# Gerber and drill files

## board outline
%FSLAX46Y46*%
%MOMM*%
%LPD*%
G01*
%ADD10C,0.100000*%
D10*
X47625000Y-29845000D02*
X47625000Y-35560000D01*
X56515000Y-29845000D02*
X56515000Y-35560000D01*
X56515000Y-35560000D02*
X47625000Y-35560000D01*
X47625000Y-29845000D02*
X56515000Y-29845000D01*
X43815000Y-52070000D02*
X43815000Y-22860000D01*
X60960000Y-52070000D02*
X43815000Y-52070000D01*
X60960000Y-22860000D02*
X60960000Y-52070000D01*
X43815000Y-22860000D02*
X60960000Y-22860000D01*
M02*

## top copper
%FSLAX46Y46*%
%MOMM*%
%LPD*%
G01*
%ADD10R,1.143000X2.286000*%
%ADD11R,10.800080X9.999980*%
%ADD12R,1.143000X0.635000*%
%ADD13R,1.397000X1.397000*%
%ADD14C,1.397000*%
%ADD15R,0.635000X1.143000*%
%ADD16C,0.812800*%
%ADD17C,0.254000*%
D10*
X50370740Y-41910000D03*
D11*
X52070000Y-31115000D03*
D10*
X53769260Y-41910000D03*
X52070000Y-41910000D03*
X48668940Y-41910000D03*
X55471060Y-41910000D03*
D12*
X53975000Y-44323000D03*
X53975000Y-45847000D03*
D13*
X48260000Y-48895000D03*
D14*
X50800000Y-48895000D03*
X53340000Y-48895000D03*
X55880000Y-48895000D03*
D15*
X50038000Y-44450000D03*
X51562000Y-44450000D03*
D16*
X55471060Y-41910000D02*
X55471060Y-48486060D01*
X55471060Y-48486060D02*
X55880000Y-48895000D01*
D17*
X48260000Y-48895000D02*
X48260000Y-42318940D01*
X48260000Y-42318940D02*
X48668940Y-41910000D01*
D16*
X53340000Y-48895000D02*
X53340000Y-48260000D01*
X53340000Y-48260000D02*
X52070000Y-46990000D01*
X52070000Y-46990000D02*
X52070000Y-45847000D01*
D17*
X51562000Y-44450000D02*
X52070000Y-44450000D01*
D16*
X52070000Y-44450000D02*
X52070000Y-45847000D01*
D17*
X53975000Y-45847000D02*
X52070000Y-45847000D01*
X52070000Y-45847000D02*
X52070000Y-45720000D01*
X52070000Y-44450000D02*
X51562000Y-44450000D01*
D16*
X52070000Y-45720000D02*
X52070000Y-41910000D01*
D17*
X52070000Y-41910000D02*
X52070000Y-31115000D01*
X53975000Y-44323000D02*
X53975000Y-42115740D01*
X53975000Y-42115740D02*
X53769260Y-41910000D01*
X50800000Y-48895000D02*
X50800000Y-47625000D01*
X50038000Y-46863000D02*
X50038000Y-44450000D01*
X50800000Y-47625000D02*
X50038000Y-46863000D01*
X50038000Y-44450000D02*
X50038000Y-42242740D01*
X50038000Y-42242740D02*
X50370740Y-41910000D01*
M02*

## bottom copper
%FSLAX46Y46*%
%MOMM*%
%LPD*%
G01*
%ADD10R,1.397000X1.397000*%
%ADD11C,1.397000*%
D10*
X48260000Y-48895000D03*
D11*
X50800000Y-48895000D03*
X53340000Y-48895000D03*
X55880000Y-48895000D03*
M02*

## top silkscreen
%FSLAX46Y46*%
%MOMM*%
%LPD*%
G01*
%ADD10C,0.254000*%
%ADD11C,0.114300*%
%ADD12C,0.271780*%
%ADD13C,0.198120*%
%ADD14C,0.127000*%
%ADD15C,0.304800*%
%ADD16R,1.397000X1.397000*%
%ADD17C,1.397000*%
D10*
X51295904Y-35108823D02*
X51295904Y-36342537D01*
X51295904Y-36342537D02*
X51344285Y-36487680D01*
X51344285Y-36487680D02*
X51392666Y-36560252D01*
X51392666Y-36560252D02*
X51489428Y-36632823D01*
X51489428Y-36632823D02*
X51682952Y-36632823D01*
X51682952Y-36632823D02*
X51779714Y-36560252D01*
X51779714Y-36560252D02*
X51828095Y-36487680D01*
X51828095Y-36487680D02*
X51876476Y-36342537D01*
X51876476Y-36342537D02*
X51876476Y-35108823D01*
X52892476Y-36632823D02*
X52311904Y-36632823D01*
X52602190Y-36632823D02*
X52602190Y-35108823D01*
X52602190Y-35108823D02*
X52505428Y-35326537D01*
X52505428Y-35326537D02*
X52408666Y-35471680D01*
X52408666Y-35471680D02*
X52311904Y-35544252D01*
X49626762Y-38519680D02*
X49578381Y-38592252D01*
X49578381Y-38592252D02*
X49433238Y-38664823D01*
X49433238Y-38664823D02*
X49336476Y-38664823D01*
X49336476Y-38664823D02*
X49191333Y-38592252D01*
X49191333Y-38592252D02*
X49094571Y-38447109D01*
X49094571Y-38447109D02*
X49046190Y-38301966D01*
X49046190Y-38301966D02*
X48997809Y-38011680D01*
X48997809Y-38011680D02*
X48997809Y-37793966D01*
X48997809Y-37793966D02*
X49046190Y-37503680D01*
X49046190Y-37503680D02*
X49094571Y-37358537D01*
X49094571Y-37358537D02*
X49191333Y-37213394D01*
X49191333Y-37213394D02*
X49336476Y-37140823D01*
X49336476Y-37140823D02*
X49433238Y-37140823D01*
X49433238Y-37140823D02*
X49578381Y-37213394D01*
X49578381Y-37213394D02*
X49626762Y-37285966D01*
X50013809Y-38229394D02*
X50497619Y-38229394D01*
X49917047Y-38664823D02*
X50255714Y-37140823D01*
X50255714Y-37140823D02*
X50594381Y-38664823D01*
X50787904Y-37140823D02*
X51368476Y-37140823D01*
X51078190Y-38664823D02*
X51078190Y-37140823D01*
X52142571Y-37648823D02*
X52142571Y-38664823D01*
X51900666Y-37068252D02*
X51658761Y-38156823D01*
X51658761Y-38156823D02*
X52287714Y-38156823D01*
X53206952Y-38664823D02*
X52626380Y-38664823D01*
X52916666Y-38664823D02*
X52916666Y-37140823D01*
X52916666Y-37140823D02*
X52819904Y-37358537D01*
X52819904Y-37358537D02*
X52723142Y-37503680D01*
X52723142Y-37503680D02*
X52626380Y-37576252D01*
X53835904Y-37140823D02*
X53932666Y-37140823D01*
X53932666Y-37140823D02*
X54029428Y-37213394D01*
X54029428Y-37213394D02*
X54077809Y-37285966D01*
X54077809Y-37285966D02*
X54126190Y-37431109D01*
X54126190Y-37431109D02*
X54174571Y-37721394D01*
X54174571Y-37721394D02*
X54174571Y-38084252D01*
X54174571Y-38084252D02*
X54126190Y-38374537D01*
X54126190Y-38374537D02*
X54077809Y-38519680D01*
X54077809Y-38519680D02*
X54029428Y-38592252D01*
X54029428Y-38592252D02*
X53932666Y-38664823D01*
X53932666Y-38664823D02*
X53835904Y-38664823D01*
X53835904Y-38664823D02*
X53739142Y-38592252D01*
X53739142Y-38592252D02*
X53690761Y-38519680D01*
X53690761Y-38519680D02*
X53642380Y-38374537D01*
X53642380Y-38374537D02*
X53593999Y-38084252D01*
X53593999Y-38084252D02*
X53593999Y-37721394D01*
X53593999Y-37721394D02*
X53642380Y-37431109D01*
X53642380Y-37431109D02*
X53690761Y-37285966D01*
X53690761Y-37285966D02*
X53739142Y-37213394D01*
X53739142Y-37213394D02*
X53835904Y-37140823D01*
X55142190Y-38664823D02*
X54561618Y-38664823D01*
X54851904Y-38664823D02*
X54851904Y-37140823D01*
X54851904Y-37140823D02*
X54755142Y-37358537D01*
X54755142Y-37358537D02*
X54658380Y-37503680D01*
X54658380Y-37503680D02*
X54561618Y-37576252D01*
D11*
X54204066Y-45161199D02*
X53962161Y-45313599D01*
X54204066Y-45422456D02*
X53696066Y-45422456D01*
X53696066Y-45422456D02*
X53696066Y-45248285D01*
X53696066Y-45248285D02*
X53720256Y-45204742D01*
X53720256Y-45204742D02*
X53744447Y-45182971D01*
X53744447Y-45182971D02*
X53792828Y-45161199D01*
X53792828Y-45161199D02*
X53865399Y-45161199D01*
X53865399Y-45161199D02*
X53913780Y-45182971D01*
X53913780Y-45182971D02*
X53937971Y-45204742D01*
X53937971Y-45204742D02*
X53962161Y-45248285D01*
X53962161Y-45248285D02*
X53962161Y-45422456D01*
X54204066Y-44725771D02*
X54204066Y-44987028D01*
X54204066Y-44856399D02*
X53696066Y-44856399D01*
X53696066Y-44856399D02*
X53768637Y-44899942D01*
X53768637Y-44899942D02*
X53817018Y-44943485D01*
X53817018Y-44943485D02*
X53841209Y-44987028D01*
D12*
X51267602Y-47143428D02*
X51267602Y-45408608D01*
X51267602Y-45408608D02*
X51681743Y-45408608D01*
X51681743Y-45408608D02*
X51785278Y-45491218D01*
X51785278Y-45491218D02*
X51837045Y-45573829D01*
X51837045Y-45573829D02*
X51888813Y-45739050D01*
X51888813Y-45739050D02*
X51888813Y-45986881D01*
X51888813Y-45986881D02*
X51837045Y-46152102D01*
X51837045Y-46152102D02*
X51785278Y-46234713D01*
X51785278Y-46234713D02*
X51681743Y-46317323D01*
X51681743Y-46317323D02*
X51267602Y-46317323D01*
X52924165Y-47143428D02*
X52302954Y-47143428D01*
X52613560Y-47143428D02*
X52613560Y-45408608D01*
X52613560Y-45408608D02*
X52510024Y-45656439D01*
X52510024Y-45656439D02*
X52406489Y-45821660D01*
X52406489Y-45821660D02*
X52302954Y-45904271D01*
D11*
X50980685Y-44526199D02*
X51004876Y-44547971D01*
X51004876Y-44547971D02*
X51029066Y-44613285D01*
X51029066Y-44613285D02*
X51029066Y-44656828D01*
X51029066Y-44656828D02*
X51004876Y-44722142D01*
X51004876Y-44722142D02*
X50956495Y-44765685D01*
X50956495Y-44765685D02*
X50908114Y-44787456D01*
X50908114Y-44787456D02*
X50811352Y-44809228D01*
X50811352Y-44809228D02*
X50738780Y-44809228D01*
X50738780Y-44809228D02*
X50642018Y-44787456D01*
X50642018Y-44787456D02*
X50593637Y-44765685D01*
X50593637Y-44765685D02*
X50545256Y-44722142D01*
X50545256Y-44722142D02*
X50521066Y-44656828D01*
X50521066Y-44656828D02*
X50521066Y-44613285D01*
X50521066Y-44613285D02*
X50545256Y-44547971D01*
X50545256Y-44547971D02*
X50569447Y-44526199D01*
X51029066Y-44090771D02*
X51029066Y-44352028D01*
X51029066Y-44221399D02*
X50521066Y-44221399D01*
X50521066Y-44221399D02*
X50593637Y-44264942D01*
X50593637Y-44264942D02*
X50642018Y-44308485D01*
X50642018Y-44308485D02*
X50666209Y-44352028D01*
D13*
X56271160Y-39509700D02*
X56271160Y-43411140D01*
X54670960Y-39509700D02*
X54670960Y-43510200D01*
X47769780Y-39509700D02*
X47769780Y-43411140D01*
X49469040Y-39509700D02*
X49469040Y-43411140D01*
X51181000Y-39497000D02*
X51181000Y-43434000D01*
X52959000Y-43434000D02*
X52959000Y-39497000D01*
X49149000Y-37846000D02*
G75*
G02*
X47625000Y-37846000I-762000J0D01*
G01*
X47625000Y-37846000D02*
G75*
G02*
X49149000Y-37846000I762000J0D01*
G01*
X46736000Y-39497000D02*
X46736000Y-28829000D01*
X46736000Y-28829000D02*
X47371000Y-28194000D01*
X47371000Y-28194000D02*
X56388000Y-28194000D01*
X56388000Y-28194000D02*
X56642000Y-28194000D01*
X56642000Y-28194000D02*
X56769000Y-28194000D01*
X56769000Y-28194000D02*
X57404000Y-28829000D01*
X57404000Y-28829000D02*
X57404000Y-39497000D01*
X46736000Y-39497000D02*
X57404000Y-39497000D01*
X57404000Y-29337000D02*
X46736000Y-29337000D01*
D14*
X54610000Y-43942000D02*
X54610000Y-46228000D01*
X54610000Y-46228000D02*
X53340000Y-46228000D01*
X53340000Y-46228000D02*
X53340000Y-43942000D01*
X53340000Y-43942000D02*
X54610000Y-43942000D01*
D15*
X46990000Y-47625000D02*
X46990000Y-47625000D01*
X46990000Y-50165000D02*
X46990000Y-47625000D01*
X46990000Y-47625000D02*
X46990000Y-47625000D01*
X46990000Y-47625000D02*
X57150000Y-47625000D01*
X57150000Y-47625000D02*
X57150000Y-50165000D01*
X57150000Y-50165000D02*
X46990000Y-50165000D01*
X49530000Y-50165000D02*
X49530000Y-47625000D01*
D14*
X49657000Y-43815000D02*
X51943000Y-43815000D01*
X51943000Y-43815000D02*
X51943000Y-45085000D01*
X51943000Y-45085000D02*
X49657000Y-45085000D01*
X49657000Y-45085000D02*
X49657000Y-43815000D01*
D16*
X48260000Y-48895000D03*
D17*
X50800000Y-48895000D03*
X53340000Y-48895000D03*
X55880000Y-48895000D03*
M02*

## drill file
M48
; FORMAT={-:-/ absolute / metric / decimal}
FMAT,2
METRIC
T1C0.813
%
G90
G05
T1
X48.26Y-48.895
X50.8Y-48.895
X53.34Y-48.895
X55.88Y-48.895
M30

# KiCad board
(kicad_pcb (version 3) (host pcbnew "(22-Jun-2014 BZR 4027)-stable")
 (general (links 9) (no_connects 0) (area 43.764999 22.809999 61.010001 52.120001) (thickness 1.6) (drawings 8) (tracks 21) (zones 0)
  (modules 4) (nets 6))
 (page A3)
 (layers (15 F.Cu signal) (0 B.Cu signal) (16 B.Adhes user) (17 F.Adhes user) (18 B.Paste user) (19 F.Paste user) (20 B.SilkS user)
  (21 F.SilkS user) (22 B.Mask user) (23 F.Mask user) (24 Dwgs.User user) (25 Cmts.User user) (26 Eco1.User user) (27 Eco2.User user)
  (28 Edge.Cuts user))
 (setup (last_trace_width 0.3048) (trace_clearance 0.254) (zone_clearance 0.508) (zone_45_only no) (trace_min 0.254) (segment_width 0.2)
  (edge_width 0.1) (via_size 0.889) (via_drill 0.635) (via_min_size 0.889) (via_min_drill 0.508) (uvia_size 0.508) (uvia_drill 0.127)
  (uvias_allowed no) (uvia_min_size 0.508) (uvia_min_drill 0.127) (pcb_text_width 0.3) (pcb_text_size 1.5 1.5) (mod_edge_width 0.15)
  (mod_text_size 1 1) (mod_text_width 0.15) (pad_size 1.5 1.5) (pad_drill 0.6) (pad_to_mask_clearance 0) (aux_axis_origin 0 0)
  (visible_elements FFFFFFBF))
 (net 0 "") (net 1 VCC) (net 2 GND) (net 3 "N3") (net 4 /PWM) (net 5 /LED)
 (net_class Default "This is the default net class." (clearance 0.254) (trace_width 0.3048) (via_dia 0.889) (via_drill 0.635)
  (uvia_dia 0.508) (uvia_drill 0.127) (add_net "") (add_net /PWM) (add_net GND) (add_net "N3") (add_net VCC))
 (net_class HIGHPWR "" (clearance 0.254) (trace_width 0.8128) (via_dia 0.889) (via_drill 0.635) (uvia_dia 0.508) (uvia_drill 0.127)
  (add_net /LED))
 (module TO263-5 (layer F.Cu) (at 52.07 41.91)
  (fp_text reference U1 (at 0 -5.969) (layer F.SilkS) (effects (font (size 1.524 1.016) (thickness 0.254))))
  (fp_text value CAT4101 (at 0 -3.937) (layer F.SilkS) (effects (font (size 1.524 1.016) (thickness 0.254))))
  (fp_line (start 4.20116 -2.4003) (end 4.20116 1.50114) (layer F.SilkS) (width 0.19812))
  (fp_line (start 2.60096 -2.4003) (end 2.60096 1.6002) (layer F.SilkS) (width 0.19812))
  (fp_line (start -4.30022 -2.4003) (end -4.30022 1.50114) (layer F.SilkS) (width 0.19812))
  (fp_line (start -2.60096 -2.4003) (end -2.60096 1.50114) (layer F.SilkS) (width 0.19812))
  (fp_line (start -0.889 -2.413) (end -0.889 1.524) (layer F.SilkS) (width 0.19812))
  (fp_line (start 0.889 1.524) (end 0.889 -2.413) (layer F.SilkS) (width 0.19812))
  (fp_circle (center -3.683 -4.064) (end -3.683 -3.302) (layer F.SilkS) (width 0.19812))
  (fp_line (start -5.334 -2.413) (end -5.334 -13.081) (layer F.SilkS) (width 0.19812))
  (fp_line (start -5.334 -13.081) (end -4.699 -13.716) (layer F.SilkS) (width 0.19812))
  (fp_line (start -4.699 -13.716) (end 4.318 -13.716) (layer F.SilkS) (width 0.19812))
  (fp_line (start 4.318 -13.716) (end 4.572 -13.716) (layer F.SilkS) (width 0.19812))
  (fp_line (start 4.572 -13.716) (end 4.699 -13.716) (layer F.SilkS) (width 0.19812))
  (fp_line (start 4.699 -13.716) (end 5.334 -13.081) (layer F.SilkS) (width 0.19812))
  (fp_line (start 5.334 -13.081) (end 5.334 -2.413) (layer F.SilkS) (width 0.19812))
  (fp_line (start -5.334 -2.413) (end 5.334 -2.413) (layer F.SilkS) (width 0.19812))
  (fp_line (start 5.334 -12.573) (end -5.334 -12.573) (layer F.SilkS) (width 0.19812))
  (pad 2 smd rect (at -1.69926 0) (size 1.143 2.286) (layers F.Cu F.Paste F.Mask) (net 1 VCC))
  (pad 3 smd rect (at 0 -10.795) (size 10.80008 9.99998) (layers F.Cu F.Paste F.Mask) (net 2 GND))
  (pad 4 smd rect (at 1.69926 0) (size 1.143 2.286) (layers F.Cu F.Paste F.Mask) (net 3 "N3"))
  (pad 3 smd rect (at 0 0) (size 1.143 2.286) (layers F.Cu F.Paste F.Mask) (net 2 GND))
  (pad 1 smd rect (at -3.40106 0) (size 1.143 2.286) (layers F.Cu F.Paste F.Mask) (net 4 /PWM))
  (pad 5 smd rect (at 3.40106 0) (size 1.143 2.286) (layers F.Cu F.Paste F.Mask) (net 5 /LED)))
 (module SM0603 (layer F.Cu) (at 53.975 45.085 270)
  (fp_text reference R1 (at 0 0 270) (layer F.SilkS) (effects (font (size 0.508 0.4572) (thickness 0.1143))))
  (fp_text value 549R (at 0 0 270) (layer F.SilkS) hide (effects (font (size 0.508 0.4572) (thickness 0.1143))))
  (fp_line (start -1.143 -0.635) (end 1.143 -0.635) (layer F.SilkS) (width 0.127))
  (fp_line (start 1.143 -0.635) (end 1.143 0.635) (layer F.SilkS) (width 0.127))
  (fp_line (start 1.143 0.635) (end -1.143 0.635) (layer F.SilkS) (width 0.127))
  (fp_line (start -1.143 0.635) (end -1.143 -0.635) (layer F.SilkS) (width 0.127))
  (pad 1 smd rect (at -0.762 0 270) (size 0.635 1.143) (layers F.Cu F.Paste F.Mask) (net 3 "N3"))
  (pad 2 smd rect (at 0.762 0 270) (size 0.635 1.143) (layers F.Cu F.Paste F.Mask) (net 2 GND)))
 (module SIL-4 (layer F.Cu) (at 52.07 48.895)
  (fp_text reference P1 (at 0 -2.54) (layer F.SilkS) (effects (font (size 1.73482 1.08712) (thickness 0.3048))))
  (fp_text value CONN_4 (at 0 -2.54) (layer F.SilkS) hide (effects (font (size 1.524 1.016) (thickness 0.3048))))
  (fp_line (start -5.08 -1.27) (end -5.08 -1.27) (layer F.SilkS) (width 0.3048))
  (fp_line (start -5.08 1.27) (end -5.08 -1.27) (layer F.SilkS) (width 0.3048))
  (fp_line (start -5.08 -1.27) (end -5.08 -1.27) (layer F.SilkS) (width 0.3048))
  (fp_line (start -5.08 -1.27) (end 5.08 -1.27) (layer F.SilkS) (width 0.3048))
  (fp_line (start 5.08 -1.27) (end 5.08 1.27) (layer F.SilkS) (width 0.3048))
  (fp_line (start 5.08 1.27) (end -5.08 1.27) (layer F.SilkS) (width 0.3048))
  (fp_line (start -2.54 1.27) (end -2.54 -1.27) (layer F.SilkS) (width 0.3048))
  (pad 1 thru_hole rect (at -3.81 0) (size 1.397 1.397) (drill 0.8128) (layers *.Cu *.Mask F.SilkS) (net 4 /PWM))
  (pad 2 thru_hole circle (at -1.27 0) (size 1.397 1.397) (drill 0.8128) (layers *.Cu *.Mask F.SilkS) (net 1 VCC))
  (pad 3 thru_hole circle (at 1.27 0) (size 1.397 1.397) (drill 0.8128) (layers *.Cu *.Mask F.SilkS) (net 2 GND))
  (pad 4 thru_hole circle (at 3.81 0) (size 1.397 1.397) (drill 0.8128) (layers *.Cu *.Mask F.SilkS) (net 5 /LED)))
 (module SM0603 (layer F.Cu) (at 50.8 44.45)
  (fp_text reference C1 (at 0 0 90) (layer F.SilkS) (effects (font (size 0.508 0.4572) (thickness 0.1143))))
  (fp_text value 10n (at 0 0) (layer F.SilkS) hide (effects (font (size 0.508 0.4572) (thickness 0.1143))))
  (fp_line (start -1.143 -0.635) (end 1.143 -0.635) (layer F.SilkS) (width 0.127))
  (fp_line (start 1.143 -0.635) (end 1.143 0.635) (layer F.SilkS) (width 0.127))
  (fp_line (start 1.143 0.635) (end -1.143 0.635) (layer F.SilkS) (width 0.127))
  (fp_line (start -1.143 0.635) (end -1.143 -0.635) (layer F.SilkS) (width 0.127))
  (pad 1 smd rect (at -0.762 0) (size 0.635 1.143) (layers F.Cu F.Paste F.Mask) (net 1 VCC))
  (pad 2 smd rect (at 0.762 0) (size 0.635 1.143) (layers F.Cu F.Paste F.Mask) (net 2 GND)))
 (gr_line (start 47.625 29.845) (end 47.625 35.56) (angle 90) (layer Edge.Cuts) (width 0.1))
 (gr_line (start 56.515 29.845) (end 56.515 35.56) (angle 90) (layer Edge.Cuts) (width 0.1))
 (gr_line (start 56.515 35.56) (end 47.625 35.56) (angle 90) (layer Edge.Cuts) (width 0.1))
 (gr_line (start 47.625 29.845) (end 56.515 29.845) (angle 90) (layer Edge.Cuts) (width 0.1))
 (gr_line (start 43.815 52.07) (end 43.815 22.86) (angle 90) (layer Edge.Cuts) (width 0.1))
 (gr_line (start 60.96 52.07) (end 43.815 52.07) (angle 90) (layer Edge.Cuts) (width 0.1))
 (gr_line (start 60.96 22.86) (end 60.96 52.07) (angle 90) (layer Edge.Cuts) (width 0.1))
 (gr_line (start 43.815 22.86) (end 60.96 22.86) (angle 90) (layer Edge.Cuts) (width 0.1))
 (segment (start 55.47106 41.91) (end 55.47106 48.48606) (width 0.8128) (layer F.Cu) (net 5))
 (segment (start 55.47106 48.48606) (end 55.88 48.895) (width 0.8128) (layer F.Cu) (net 5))
 (segment (start 48.26 48.895) (end 48.26 42.31894) (width 0.254) (layer F.Cu) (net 4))
 (segment (start 48.26 42.31894) (end 48.66894 41.91) (width 0.254) (layer F.Cu) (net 4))
 (segment (start 53.34 48.895) (end 53.34 48.26) (width 0.8128) (layer F.Cu) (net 2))
 (segment (start 53.34 48.26) (end 52.07 46.99) (width 0.8128) (layer F.Cu) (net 2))
 (segment (start 52.07 46.99) (end 52.07 45.847) (width 0.8128) (layer F.Cu) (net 2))
 (segment (start 51.562 44.45) (end 52.07 44.45) (width 0.254) (layer F.Cu) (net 2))
 (segment (start 52.07 44.45) (end 52.07 45.847) (width 0.8128) (layer F.Cu) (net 2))
 (segment (start 53.975 45.847) (end 52.07 45.847) (width 0.254) (layer F.Cu) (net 2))
 (segment (start 52.07 45.847) (end 52.07 45.72) (width 0.254) (layer F.Cu) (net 2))
 (segment (start 52.07 44.45) (end 51.562 44.45) (width 0.254) (layer F.Cu) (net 2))
 (segment (start 52.07 45.72) (end 52.07 41.91) (width 0.8128) (layer F.Cu) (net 2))
 (segment (start 52.07 41.91) (end 52.07 31.115) (width 0.254) (layer F.Cu) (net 2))
 (segment (start 53.975 44.323) (end 53.975 42.11574) (width 0.254) (layer F.Cu) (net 3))
 (segment (start 53.975 42.11574) (end 53.76926 41.91) (width 0.254) (layer F.Cu) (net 3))
 (segment (start 50.8 48.895) (end 50.8 47.625) (width 0.254) (layer F.Cu) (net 1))
 (segment (start 50.038 46.863) (end 50.038 44.45) (width 0.254) (layer F.Cu) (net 1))
 (segment (start 50.8 47.625) (end 50.038 46.863) (width 0.254) (layer F.Cu) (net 1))
 (segment (start 50.038 44.45) (end 50.038 42.24274) (width 0.254) (layer F.Cu) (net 1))
 (segment (start 50.038 42.24274) (end 50.37074 41.91) (width 0.254) (layer F.Cu) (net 1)))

